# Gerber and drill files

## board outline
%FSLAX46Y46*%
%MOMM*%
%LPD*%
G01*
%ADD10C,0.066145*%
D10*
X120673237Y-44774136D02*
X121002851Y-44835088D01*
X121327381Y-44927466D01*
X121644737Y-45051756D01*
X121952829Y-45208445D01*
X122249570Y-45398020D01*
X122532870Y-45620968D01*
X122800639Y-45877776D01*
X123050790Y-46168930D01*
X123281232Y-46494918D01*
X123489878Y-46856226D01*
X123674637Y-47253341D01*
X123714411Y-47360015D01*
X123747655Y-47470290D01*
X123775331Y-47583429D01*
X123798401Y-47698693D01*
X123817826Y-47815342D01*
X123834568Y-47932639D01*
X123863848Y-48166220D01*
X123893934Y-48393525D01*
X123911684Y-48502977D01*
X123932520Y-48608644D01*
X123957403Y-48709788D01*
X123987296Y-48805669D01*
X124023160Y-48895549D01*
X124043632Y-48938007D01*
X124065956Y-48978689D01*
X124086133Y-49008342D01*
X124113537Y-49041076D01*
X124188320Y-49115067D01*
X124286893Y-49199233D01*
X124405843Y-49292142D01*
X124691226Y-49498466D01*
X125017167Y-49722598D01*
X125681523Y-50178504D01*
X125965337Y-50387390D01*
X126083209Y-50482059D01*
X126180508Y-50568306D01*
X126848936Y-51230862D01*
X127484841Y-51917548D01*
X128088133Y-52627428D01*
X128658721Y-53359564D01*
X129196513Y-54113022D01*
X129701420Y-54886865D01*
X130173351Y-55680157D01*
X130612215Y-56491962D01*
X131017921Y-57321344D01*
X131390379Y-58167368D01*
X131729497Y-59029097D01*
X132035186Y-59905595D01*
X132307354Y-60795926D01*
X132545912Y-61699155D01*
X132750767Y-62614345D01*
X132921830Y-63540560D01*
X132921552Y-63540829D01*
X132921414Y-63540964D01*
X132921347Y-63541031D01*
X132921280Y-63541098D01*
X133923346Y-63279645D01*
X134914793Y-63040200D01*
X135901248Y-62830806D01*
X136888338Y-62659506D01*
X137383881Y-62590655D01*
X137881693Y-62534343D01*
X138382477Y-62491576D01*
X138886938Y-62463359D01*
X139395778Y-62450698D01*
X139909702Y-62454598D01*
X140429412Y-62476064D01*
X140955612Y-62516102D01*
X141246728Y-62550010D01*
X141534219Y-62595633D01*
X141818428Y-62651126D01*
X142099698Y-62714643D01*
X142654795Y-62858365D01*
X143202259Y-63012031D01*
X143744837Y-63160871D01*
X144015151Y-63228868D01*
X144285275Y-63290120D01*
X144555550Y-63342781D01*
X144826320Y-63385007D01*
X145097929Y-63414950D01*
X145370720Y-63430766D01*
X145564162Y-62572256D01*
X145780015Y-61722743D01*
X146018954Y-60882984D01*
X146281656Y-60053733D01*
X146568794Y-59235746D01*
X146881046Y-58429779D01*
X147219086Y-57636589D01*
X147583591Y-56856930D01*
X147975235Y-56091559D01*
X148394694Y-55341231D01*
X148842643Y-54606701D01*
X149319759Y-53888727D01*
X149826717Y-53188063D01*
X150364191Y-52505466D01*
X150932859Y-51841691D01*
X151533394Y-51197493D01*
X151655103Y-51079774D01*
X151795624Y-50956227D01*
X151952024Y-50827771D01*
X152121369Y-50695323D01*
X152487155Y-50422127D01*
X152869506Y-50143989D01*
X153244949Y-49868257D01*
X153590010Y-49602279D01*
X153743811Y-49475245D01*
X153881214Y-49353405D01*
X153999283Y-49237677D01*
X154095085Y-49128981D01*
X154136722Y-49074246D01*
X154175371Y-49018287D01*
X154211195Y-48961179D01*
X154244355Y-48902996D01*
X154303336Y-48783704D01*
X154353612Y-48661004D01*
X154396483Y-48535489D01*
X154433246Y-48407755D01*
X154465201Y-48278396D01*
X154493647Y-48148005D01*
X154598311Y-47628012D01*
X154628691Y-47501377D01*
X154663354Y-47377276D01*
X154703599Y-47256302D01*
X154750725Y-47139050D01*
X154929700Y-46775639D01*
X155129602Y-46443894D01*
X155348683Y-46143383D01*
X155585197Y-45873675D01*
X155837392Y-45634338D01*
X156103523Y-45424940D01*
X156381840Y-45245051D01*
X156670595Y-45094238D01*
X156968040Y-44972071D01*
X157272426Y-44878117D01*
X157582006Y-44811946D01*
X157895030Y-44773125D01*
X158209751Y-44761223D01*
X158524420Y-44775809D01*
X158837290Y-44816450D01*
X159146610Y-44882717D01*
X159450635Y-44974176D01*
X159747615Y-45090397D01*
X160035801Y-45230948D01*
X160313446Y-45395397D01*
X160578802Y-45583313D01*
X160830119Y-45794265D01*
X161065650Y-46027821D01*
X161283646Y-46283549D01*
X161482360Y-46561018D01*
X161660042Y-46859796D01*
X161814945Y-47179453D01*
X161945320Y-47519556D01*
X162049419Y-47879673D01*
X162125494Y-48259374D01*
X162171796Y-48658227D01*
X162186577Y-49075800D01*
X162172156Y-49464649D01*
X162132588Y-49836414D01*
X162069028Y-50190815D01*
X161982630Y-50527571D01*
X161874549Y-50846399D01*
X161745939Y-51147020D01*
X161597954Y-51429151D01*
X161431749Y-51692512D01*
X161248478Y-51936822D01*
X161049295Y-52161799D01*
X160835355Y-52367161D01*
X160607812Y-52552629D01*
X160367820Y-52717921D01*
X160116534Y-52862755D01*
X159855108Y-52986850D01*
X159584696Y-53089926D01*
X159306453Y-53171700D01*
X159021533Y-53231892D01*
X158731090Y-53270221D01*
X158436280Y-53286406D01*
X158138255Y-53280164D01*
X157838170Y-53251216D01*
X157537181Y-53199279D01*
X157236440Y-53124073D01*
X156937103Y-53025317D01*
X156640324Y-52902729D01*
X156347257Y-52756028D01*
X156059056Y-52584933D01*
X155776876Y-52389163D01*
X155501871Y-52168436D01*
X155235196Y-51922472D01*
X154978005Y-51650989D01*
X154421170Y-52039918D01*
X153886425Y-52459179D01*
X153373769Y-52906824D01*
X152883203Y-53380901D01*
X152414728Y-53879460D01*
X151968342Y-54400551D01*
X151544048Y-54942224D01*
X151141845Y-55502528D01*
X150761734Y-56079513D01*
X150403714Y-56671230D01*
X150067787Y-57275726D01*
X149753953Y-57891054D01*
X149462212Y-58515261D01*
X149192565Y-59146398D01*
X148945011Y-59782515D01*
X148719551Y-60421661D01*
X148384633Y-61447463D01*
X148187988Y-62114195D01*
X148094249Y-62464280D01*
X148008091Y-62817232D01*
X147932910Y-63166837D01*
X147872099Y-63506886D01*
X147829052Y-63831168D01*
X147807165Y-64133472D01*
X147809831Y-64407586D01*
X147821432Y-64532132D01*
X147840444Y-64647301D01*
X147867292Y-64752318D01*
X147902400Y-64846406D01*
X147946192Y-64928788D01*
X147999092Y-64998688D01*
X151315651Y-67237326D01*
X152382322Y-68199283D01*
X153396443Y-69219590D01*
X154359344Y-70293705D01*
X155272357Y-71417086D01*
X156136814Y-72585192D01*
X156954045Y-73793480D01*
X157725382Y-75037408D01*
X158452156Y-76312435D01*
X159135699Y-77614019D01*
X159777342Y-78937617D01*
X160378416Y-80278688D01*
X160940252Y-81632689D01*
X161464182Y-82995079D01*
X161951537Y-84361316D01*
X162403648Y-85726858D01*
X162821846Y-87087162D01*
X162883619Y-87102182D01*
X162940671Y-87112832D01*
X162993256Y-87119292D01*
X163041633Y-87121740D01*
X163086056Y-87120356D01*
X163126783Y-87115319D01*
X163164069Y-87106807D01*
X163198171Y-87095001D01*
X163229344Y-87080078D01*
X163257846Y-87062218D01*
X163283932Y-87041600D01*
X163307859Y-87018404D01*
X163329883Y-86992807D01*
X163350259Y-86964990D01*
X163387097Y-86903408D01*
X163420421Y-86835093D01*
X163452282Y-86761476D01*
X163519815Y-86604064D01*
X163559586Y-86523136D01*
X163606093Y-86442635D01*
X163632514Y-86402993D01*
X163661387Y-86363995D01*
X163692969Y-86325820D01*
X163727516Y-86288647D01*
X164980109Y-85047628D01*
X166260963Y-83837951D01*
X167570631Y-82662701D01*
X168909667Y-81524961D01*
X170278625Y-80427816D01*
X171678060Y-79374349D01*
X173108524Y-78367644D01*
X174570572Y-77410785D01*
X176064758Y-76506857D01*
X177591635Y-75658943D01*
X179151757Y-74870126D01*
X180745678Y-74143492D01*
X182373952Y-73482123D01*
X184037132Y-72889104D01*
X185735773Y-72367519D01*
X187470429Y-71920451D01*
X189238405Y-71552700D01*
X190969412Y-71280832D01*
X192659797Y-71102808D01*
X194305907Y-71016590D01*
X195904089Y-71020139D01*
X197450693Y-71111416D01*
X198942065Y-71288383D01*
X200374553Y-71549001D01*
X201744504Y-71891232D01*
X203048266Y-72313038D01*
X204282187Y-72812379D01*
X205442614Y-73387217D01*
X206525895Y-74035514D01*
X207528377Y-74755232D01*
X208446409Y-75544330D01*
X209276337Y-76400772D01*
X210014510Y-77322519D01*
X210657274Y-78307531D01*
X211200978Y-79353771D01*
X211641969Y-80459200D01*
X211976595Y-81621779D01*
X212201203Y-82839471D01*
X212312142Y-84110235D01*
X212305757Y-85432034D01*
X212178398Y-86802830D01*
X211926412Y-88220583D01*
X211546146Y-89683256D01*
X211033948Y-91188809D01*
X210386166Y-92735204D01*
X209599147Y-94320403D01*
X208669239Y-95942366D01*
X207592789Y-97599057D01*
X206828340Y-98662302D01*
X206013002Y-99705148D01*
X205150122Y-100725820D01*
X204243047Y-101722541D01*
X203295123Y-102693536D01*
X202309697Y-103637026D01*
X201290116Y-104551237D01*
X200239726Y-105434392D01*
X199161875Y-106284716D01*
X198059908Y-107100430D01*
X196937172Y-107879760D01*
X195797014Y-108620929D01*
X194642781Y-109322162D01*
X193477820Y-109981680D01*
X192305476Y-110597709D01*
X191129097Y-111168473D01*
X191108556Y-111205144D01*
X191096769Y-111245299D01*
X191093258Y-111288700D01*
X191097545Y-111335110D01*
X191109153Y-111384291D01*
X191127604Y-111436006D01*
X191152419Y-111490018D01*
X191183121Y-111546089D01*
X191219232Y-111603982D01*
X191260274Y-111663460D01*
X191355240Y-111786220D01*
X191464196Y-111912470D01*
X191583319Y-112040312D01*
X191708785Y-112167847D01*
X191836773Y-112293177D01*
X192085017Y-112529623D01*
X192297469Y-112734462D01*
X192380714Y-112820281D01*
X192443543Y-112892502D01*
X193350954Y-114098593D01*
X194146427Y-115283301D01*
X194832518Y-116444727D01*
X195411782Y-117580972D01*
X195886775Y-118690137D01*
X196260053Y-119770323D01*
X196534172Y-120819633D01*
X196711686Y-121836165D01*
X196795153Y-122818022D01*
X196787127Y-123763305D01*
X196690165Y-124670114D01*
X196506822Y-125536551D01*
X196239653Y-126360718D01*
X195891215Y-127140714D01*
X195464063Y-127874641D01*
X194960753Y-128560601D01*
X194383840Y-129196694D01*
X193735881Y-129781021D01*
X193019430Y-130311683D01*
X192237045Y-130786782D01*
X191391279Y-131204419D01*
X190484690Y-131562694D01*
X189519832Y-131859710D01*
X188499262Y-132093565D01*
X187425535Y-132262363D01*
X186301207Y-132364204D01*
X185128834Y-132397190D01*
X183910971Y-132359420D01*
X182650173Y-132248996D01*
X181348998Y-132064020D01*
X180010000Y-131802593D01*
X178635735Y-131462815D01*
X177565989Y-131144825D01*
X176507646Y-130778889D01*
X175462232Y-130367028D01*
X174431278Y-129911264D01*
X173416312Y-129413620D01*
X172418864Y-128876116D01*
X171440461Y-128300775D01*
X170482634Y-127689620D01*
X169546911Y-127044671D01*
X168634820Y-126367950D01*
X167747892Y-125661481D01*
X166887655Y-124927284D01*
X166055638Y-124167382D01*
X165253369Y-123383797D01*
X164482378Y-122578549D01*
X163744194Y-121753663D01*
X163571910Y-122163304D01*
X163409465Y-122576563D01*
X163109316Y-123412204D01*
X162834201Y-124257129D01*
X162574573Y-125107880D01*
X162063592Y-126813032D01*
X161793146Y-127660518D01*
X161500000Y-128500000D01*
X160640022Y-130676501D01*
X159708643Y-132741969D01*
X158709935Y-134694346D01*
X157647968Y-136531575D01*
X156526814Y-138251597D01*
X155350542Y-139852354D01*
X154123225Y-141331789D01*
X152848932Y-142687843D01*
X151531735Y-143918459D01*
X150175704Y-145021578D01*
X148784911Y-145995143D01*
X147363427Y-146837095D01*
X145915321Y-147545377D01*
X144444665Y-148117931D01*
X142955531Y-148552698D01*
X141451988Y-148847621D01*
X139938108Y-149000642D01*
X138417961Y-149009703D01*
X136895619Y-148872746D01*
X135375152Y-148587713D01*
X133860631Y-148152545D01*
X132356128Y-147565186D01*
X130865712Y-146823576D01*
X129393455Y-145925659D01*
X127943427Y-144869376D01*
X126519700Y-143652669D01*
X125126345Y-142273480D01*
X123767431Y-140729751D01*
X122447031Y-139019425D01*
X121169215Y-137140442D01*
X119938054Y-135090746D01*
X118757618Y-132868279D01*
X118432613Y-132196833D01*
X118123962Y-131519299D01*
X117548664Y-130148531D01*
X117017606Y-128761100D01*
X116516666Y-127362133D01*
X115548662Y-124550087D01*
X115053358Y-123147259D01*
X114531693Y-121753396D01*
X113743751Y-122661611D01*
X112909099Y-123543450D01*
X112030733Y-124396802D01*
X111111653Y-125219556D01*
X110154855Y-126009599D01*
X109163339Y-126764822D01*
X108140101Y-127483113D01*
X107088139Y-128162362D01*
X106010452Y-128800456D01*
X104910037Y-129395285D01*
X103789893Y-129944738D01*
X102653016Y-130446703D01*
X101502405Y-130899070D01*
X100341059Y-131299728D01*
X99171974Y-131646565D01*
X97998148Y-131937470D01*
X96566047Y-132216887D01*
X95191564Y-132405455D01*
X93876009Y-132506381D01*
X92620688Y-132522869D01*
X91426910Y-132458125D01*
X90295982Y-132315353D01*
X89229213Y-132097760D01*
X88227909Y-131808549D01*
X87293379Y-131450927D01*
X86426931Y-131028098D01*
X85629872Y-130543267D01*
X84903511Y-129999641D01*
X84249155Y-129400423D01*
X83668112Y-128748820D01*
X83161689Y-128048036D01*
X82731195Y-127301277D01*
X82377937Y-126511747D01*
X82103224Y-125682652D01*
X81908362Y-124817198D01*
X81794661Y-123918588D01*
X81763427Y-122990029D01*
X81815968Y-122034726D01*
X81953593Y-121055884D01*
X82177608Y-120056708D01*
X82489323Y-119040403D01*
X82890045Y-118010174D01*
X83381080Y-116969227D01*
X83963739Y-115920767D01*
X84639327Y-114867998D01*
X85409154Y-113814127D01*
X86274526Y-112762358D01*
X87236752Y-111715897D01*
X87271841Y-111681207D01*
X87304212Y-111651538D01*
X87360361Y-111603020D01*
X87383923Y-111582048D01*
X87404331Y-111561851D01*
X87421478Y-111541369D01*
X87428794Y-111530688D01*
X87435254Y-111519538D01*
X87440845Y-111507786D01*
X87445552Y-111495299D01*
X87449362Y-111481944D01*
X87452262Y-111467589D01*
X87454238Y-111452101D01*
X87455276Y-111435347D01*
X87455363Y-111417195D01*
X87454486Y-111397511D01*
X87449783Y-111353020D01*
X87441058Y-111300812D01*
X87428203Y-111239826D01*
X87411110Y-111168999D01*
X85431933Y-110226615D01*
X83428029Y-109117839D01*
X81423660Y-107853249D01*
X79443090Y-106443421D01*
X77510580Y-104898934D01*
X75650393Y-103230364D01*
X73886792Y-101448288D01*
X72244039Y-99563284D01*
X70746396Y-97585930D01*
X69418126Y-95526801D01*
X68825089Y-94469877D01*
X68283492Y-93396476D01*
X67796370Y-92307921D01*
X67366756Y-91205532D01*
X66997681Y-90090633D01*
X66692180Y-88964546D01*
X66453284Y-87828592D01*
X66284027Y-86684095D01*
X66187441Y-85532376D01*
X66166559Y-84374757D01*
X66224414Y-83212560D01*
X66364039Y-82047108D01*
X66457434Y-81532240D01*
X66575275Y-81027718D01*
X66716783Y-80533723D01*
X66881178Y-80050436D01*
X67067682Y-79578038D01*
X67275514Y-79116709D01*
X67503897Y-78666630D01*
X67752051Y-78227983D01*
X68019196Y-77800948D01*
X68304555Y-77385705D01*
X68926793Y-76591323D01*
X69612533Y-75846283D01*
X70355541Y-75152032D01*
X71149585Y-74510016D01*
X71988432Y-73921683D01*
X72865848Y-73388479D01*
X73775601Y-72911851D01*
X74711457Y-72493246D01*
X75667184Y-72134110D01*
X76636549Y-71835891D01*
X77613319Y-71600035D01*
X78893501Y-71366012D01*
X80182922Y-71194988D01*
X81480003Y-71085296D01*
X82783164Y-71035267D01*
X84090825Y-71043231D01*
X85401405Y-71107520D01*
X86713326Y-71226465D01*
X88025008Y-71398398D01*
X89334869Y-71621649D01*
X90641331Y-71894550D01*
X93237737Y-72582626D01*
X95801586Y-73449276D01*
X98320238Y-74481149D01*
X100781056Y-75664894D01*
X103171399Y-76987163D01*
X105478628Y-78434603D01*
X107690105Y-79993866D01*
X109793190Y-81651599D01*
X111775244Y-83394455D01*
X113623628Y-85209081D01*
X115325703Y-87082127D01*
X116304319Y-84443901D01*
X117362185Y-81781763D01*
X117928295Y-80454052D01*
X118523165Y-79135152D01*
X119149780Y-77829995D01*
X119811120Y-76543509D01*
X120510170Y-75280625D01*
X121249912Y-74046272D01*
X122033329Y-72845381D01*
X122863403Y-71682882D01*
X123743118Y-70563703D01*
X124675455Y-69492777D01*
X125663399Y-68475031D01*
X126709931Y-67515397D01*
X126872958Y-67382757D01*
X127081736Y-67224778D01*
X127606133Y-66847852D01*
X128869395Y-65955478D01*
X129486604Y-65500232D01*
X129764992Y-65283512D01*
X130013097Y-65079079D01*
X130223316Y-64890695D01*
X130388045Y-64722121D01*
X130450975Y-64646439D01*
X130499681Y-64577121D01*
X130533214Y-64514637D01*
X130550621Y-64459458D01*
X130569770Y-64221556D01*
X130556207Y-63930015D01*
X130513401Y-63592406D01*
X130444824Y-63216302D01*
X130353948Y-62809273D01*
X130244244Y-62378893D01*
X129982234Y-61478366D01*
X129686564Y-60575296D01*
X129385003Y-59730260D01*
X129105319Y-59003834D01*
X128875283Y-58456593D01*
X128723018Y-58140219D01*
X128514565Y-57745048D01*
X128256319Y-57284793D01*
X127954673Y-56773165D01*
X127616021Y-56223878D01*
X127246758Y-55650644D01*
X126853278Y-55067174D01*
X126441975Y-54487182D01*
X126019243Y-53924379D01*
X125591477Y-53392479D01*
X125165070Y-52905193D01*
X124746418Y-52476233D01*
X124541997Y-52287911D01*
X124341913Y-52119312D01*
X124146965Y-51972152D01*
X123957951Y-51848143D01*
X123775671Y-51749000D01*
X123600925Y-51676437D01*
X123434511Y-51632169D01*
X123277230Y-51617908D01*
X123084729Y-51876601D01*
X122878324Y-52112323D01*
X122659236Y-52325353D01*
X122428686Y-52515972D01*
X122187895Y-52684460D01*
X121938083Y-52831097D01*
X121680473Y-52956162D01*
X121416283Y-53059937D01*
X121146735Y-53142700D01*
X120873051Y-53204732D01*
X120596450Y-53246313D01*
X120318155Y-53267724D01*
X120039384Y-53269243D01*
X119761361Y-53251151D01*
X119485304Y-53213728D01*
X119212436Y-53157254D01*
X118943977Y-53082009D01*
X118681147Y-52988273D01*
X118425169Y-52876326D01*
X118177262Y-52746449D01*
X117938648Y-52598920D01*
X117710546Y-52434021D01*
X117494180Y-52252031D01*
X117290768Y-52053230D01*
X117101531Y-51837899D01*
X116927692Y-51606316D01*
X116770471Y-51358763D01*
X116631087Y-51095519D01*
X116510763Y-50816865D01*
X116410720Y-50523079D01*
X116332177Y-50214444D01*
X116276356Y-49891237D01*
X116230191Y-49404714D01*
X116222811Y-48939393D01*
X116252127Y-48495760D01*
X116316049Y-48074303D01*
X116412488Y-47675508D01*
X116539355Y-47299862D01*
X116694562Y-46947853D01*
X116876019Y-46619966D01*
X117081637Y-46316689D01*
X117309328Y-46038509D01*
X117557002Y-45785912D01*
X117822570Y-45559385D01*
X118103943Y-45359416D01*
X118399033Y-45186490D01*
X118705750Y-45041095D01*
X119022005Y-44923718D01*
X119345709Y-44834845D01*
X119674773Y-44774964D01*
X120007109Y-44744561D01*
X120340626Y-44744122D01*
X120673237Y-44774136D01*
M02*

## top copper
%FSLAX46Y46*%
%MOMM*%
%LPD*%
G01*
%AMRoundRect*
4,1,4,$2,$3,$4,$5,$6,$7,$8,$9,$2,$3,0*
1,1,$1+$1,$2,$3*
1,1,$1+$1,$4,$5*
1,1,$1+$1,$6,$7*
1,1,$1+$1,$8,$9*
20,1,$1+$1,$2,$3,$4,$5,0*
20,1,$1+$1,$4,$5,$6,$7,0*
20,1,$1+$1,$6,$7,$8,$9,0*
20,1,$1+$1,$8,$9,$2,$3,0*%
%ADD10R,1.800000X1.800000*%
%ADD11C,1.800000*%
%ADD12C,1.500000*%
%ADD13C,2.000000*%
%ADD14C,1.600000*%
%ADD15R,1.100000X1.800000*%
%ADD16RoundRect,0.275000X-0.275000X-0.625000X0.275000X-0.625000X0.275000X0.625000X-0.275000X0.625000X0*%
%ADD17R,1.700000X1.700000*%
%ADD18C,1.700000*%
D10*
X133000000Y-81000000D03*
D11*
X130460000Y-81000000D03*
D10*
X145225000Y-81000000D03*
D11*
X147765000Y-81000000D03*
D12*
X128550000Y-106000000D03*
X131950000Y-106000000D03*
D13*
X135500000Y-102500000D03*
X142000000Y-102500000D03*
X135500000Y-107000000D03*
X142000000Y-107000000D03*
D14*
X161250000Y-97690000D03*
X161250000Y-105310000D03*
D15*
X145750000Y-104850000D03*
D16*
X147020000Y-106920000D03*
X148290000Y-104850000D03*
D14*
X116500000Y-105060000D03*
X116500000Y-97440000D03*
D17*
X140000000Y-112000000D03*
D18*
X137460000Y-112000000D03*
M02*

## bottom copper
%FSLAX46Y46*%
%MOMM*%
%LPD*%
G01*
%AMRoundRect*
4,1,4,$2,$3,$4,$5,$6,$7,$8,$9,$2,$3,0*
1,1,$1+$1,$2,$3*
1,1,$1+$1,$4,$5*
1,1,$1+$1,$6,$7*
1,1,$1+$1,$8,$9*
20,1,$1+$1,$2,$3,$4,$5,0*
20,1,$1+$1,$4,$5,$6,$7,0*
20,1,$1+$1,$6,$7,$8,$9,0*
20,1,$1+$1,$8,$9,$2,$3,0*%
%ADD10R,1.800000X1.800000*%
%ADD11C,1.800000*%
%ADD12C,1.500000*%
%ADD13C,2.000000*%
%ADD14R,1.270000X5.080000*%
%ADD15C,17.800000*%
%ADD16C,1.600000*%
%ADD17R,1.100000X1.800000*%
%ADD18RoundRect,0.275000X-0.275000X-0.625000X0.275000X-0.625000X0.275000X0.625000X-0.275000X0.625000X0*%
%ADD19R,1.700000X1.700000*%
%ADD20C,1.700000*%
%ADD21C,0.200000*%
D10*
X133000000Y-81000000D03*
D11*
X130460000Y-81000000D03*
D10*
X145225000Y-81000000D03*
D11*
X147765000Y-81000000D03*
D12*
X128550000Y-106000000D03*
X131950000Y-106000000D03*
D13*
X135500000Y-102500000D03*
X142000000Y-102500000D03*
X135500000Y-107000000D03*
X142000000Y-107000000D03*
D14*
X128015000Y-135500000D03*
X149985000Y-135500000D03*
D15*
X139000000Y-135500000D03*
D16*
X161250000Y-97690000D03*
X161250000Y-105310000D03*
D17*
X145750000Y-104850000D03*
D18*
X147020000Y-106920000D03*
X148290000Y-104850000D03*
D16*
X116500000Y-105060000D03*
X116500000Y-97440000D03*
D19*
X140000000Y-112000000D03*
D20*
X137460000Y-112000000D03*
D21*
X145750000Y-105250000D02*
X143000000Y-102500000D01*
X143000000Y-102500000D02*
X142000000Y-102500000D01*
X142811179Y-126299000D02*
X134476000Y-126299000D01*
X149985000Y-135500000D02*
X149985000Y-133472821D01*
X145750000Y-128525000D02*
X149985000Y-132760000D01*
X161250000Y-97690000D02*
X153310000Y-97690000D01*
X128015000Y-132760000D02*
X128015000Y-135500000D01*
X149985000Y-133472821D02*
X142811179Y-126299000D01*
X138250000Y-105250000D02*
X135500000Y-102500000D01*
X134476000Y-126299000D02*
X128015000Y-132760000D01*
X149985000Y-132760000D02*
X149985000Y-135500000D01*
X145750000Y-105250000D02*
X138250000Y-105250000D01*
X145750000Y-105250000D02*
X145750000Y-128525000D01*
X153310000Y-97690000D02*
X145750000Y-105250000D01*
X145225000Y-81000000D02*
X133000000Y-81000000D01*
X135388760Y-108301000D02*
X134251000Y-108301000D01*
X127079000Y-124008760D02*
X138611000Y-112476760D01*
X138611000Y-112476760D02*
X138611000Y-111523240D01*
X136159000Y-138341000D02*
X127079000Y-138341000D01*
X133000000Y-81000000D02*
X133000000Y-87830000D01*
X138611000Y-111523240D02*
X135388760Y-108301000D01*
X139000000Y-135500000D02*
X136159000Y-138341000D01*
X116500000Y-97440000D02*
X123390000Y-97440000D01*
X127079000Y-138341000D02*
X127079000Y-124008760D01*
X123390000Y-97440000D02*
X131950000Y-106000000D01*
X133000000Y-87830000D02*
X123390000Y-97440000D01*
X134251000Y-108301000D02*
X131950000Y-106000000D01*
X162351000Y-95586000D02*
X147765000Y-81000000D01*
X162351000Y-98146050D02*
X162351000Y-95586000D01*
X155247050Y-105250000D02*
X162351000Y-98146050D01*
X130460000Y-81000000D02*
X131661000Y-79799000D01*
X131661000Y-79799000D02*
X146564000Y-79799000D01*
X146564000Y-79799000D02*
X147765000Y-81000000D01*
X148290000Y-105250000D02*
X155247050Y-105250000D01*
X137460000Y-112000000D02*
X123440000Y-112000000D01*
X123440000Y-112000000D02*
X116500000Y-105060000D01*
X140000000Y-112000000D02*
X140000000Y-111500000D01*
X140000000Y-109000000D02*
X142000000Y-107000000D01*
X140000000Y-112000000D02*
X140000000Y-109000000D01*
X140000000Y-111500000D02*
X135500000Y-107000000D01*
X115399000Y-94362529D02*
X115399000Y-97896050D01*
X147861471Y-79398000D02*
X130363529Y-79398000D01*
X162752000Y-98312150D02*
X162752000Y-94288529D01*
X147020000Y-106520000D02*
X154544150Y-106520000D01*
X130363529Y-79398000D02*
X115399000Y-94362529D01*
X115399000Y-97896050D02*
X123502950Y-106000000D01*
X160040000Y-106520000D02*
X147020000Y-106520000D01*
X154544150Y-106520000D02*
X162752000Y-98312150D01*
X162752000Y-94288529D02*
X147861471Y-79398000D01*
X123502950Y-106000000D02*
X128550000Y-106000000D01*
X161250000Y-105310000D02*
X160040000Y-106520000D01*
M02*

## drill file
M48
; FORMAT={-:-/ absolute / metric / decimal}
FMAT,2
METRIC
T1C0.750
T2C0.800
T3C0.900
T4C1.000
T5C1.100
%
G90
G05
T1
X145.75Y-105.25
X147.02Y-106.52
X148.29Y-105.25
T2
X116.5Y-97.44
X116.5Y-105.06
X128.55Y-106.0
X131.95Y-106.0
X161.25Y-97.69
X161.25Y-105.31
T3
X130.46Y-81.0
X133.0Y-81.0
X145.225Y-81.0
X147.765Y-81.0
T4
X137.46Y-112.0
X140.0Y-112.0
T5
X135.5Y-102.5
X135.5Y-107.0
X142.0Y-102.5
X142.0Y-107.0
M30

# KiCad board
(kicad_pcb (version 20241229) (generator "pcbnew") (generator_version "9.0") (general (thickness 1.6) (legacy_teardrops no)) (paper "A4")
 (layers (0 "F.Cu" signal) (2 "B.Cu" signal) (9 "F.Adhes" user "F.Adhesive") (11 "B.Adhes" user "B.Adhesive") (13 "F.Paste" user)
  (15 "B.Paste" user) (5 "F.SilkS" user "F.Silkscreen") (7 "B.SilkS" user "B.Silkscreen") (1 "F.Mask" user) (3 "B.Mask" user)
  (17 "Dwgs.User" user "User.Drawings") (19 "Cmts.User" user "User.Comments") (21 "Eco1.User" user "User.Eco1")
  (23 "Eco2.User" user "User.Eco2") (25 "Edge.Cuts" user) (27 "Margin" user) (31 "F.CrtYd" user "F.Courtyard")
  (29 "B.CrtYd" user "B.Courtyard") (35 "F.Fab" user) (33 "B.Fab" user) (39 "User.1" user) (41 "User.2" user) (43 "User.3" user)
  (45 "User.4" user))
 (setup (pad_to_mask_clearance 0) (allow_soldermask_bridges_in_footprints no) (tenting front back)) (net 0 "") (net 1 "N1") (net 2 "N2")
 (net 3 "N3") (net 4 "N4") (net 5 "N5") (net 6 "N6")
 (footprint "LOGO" (layer "F.Cu") (at 139.25 97.25)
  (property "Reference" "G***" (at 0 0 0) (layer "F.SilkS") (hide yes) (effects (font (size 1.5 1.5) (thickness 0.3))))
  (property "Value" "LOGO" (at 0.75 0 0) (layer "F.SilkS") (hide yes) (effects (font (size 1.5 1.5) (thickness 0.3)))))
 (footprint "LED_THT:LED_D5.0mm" (layer "F.Cu") (at 133 81 180)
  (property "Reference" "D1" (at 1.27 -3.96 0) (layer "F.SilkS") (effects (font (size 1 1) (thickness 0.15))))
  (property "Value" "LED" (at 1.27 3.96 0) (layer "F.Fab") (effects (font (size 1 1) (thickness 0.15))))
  (pad "1" thru_hole rect (at 0 0 180) (size 1.8 1.8) (drill 0.9) (layers "*.Cu" "*.Mask") (remove_unused_layers no) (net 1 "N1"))
  (pad "2" thru_hole circle (at 2.54 0 180) (size 1.8 1.8) (drill 0.9) (layers "*.Cu" "*.Mask") (remove_unused_layers no) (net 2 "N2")))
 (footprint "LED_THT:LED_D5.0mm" (layer "F.Cu") (at 145.225 81)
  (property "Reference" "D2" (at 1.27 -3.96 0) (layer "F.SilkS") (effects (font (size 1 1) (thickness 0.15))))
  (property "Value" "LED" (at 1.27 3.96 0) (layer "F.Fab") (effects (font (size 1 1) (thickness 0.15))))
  (pad "1" thru_hole rect (at 0 0) (size 1.8 1.8) (drill 0.9) (layers "*.Cu" "*.Mask") (remove_unused_layers no) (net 1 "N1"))
  (pad "2" thru_hole circle (at 2.54 0) (size 1.8 1.8) (drill 0.9) (layers "*.Cu" "*.Mask") (remove_unused_layers no) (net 2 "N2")))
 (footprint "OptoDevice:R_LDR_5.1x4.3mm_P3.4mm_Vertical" (layer "F.Cu") (at 128.55 106)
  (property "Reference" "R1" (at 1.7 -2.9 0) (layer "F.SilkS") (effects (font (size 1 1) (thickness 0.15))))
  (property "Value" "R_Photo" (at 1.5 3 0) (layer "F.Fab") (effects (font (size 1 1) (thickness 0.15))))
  (pad "1" thru_hole circle (at 0 0) (size 1.5 1.5) (drill 0.8) (layers "*.Cu" "*.Mask") (remove_unused_layers no) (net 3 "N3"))
  (pad "2" thru_hole circle (at 3.4 0) (size 1.5 1.5) (drill 0.8) (layers "*.Cu" "*.Mask") (remove_unused_layers no) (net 1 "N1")))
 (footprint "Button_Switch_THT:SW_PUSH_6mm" (layer "F.Cu") (at 135.5 102.5)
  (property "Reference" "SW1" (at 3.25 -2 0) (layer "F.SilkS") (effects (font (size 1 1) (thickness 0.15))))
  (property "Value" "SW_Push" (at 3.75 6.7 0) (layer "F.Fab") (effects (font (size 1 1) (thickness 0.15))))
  (pad "1" thru_hole circle (at 0 0 90) (size 2 2) (drill 1.1) (layers "*.Cu" "*.Mask") (remove_unused_layers no) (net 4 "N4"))
  (pad "1" thru_hole circle (at 6.5 0 90) (size 2 2) (drill 1.1) (layers "*.Cu" "*.Mask") (remove_unused_layers no) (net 4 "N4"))
  (pad "2" thru_hole circle (at 0 4.5 90) (size 2 2) (drill 1.1) (layers "*.Cu" "*.Mask") (remove_unused_layers no) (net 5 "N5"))
  (pad "2" thru_hole circle (at 6.5 4.5 90) (size 2 2) (drill 1.1) (layers "*.Cu" "*.Mask") (remove_unused_layers no) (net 5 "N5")))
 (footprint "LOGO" (layer "B.Cu") (at 102.5 124 180)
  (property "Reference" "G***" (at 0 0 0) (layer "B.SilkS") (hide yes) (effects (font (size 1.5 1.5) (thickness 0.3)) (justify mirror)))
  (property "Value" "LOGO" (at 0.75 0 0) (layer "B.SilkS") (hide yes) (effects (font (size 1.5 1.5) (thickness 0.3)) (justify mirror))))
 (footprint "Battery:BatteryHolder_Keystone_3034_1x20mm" (layer "B.Cu") (at 139 135.5)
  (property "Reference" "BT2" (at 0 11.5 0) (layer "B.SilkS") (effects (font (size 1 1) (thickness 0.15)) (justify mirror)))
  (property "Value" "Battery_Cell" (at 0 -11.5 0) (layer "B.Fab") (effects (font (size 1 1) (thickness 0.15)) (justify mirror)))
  (pad "1" smd rect (at -10.985 0) (size 1.27 5.08) (layers "B.Cu" "B.Mask" "B.Paste") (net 4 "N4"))
  (pad "1" smd rect (at 10.985 0) (size 1.27 5.08) (layers "B.Cu" "B.Mask" "B.Paste") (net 4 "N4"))
  (pad "2" smd circle (at 0 0) (size 17.8 17.8) (layers "B.Cu" "B.Mask") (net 1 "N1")))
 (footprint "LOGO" (layer "B.Cu") (at 183.5 123.75 180)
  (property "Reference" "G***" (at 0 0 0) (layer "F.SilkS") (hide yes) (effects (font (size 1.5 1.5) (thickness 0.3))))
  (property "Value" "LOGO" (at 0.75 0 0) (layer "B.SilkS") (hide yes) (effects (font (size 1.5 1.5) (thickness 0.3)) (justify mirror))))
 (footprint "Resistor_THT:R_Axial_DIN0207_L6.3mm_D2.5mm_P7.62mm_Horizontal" (layer "B.Cu") (at 161.25 97.69 -90)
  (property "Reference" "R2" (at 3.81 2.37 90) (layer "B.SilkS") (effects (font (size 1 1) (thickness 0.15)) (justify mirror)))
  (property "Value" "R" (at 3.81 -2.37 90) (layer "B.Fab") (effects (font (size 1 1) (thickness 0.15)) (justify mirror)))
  (pad "1" thru_hole circle (at 0 0 270) (size 1.6 1.6) (drill 0.8) (layers "*.Cu" "*.Mask") (remove_unused_layers no) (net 4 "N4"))
  (pad "2" thru_hole circle (at 7.62 0 270) (size 1.6 1.6) (drill 0.8) (layers "*.Cu" "*.Mask") (remove_unused_layers no) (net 3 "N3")))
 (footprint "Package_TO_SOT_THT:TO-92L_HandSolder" (layer "B.Cu") (at 145.75 105.25)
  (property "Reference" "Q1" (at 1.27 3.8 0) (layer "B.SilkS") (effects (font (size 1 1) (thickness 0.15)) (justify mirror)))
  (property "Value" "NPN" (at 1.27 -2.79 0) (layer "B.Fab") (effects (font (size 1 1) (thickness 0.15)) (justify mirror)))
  (pad "1" thru_hole rect (at 0 0) (size 1.1 1.8) (drill 0.75 (offset 0 -0.4)) (layers "*.Cu" "*.Mask") (remove_unused_layers no)
   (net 4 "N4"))
  (pad "2" thru_hole roundrect (at 1.27 1.27) (size 1.1 1.8) (drill 0.75 (offset 0 0.4)) (layers "*.Cu" "*.Mask") (remove_unused_layers no)
   (roundrect_rratio 0.25) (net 3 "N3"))
  (pad "3" thru_hole roundrect (at 2.54 0) (size 1.1 1.8) (drill 0.75 (offset 0 -0.4)) (layers "*.Cu" "*.Mask") (remove_unused_layers no)
   (roundrect_rratio 0.25) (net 2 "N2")))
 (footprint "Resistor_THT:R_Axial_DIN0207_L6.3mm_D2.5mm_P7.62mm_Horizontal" (layer "B.Cu") (at 116.5 105.06 90)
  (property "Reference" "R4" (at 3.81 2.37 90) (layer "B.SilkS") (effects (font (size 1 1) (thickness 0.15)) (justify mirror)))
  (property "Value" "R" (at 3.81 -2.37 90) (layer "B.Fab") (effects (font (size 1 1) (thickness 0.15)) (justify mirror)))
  (pad "1" thru_hole circle (at 0 0 90) (size 1.6 1.6) (drill 0.8) (layers "*.Cu" "*.Mask") (remove_unused_layers no) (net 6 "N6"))
  (pad "2" thru_hole circle (at 7.62 0 90) (size 1.6 1.6) (drill 0.8) (layers "*.Cu" "*.Mask") (remove_unused_layers no) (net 1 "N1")))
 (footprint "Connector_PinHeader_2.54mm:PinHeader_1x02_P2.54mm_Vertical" (layer "B.Cu") (at 140 112 90)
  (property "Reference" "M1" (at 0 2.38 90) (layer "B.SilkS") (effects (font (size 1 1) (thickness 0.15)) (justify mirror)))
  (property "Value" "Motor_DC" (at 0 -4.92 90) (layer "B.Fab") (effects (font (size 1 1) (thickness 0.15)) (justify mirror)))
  (pad "1" thru_hole rect (at 0 0 90) (size 1.7 1.7) (drill 1) (layers "*.Cu" "*.Mask") (remove_unused_layers no) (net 5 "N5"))
  (pad "2" thru_hole circle (at 0 -2.54 90) (size 1.7 1.7) (drill 1) (layers "*.Cu" "*.Mask") (remove_unused_layers no) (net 6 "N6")))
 (gr_poly
  (pts (xy 120.673237 44.774136) (xy 121.002851 44.835088) (xy 121.327381 44.927466) (xy 121.644737 45.051756) (xy 121.952829 45.208445)
   (xy 122.24957 45.39802) (xy 122.53287 45.620968) (xy 122.800639 45.877776) (xy 123.05079 46.16893) (xy 123.281232 46.494918)
   (xy 123.489878 46.856226) (xy 123.674637 47.253341) (xy 123.714411 47.360015) (xy 123.747655 47.47029) (xy 123.775331 47.583429)
   (xy 123.798401 47.698693) (xy 123.817826 47.815342) (xy 123.834568 47.932639) (xy 123.863848 48.16622) (xy 123.893934 48.393525)
   (xy 123.911684 48.502977) (xy 123.93252 48.608644) (xy 123.957403 48.709788) (xy 123.987296 48.805669) (xy 124.02316 48.895549)
   (xy 124.043632 48.938007) (xy 124.065956 48.978689) (xy 124.086133 49.008342) (xy 124.113537 49.041076) (xy 124.18832 49.115067)
   (xy 124.286893 49.199233) (xy 124.405843 49.292142) (xy 124.691226 49.498466) (xy 125.017167 49.722598) (xy 125.681523 50.178504)
   (xy 125.965337 50.38739) (xy 126.083209 50.482059) (xy 126.180508 50.568306) (xy 126.848936 51.230862) (xy 127.484841 51.917548)
   (xy 128.088133 52.627428) (xy 128.658721 53.359564) (xy 129.196513 54.113022) (xy 129.70142 54.886865) (xy 130.173351 55.680157)
   (xy 130.612215 56.491962) (xy 131.017921 57.321344) (xy 131.390379 58.167368) (xy 131.729497 59.029097) (xy 132.035186 59.905595)
   (xy 132.307354 60.795926) (xy 132.545912 61.699155) (xy 132.750767 62.614345) (xy 132.92183 63.54056) (xy 132.921552 63.540829)
   (xy 132.921414 63.540964) (xy 132.921347 63.541031) (xy 132.92128 63.541098) (xy 133.923346 63.279645) (xy 134.914793 63.0402)
   (xy 135.901248 62.830806) (xy 136.888338 62.659506) (xy 137.383881 62.590655) (xy 137.881693 62.534343) (xy 138.382477 62.491576)
   (xy 138.886938 62.463359) (xy 139.395778 62.450698) (xy 139.909702 62.454598) (xy 140.429412 62.476064) (xy 140.955612 62.516102)
   (xy 141.246728 62.55001) (xy 141.534219 62.595633) (xy 141.818428 62.651126) (xy 142.099698 62.714643) (xy 142.654795 62.858365)
   (xy 143.202259 63.012031) (xy 143.744837 63.160871) (xy 144.015151 63.228868) (xy 144.285275 63.29012) (xy 144.55555 63.342781)
   (xy 144.82632 63.385007) (xy 145.097929 63.41495) (xy 145.37072 63.430766) (xy 145.564162 62.572256) (xy 145.780015 61.722743)
   (xy 146.018954 60.882984) (xy 146.281656 60.053733) (xy 146.568794 59.235746) (xy 146.881046 58.429779) (xy 147.219086 57.636589)
   (xy 147.583591 56.85693) (xy 147.975235 56.091559) (xy 148.394694 55.341231) (xy 148.842643 54.606701) (xy 149.319759 53.888727)
   (xy 149.826717 53.188063) (xy 150.364191 52.505466) (xy 150.932859 51.841691) (xy 151.533394 51.197493) (xy 151.655103 51.079774)
   (xy 151.795624 50.956227) (xy 151.952024 50.827771) (xy 152.121369 50.695323) (xy 152.487155 50.422127) (xy 152.869506 50.143989)
   (xy 153.244949 49.868257) (xy 153.59001 49.602279) (xy 153.743811 49.475245) (xy 153.881214 49.353405) (xy 153.999283 49.237677)
   (xy 154.095085 49.128981) (xy 154.136722 49.074246) (xy 154.175371 49.018287) (xy 154.211195 48.961179) (xy 154.244355 48.902996)
   (xy 154.303336 48.783704) (xy 154.353612 48.661004) (xy 154.396483 48.535489) (xy 154.433246 48.407755) (xy 154.465201 48.278396)
   (xy 154.493647 48.148005) (xy 154.598311 47.628012) (xy 154.628691 47.501377) (xy 154.663354 47.377276) (xy 154.703599 47.256302)
   (xy 154.750725 47.13905) (xy 154.9297 46.775639) (xy 155.129602 46.443894) (xy 155.348683 46.143383) (xy 155.585197 45.873675)
   (xy 155.837392 45.634338) (xy 156.103523 45.42494) (xy 156.38184 45.245051) (xy 156.670595 45.094238) (xy 156.96804 44.972071)
   (xy 157.272426 44.878117) (xy 157.582006 44.811946) (xy 157.89503 44.773125) (xy 158.209751 44.761223) (xy 158.52442 44.775809)
   (xy 158.83729 44.81645) (xy 159.14661 44.882717) (xy 159.450635 44.974176) (xy 159.747615 45.090397) (xy 160.035801 45.230948)
   (xy 160.313446 45.395397) (xy 160.578802 45.583313) (xy 160.830119 45.794265) (xy 161.06565 46.027821) (xy 161.283646 46.283549)
   (xy 161.48236 46.561018) (xy 161.660042 46.859796) (xy 161.814945 47.179453) (xy 161.94532 47.519556) (xy 162.049419 47.879673)
   (xy 162.125494 48.259374) (xy 162.171796 48.658227) (xy 162.186577 49.0758) (xy 162.172156 49.464649) (xy 162.132588 49.836414)
   (xy 162.069028 50.190815) (xy 161.98263 50.527571) (xy 161.874549 50.846399) (xy 161.745939 51.14702) (xy 161.597954 51.429151)
   (xy 161.431749 51.692512) (xy 161.248478 51.936822) (xy 161.049295 52.161799) (xy 160.835355 52.367161) (xy 160.607812 52.552629)
   (xy 160.36782 52.717921) (xy 160.116534 52.862755) (xy 159.855108 52.98685) (xy 159.584696 53.089926) (xy 159.306453 53.1717)
   (xy 159.021533 53.231892) (xy 158.73109 53.270221) (xy 158.43628 53.286406) (xy 158.138255 53.280164) (xy 157.83817 53.251216)
   (xy 157.537181 53.199279) (xy 157.23644 53.124073) (xy 156.937103 53.025317) (xy 156.640324 52.902729) (xy 156.347257 52.756028)
   (xy 156.059056 52.584933) (xy 155.776876 52.389163) (xy 155.501871 52.168436) (xy 155.235196 51.922472) (xy 154.978005 51.650989)
   (xy 154.42117 52.039918) (xy 153.886425 52.459179) (xy 153.373769 52.906824) (xy 152.883203 53.380901) (xy 152.414728 53.87946)
   (xy 151.968342 54.400551) (xy 151.544048 54.942224) (xy 151.141845 55.502528) (xy 150.761734 56.079513) (xy 150.403714 56.67123)
   (xy 150.067787 57.275726) (xy 149.753953 57.891054) (xy 149.462212 58.515261) (xy 149.192565 59.146398) (xy 148.945011 59.782515)
   (xy 148.719551 60.421661) (xy 148.384633 61.447463) (xy 148.187988 62.114195) (xy 148.094249 62.46428) (xy 148.008091 62.817232)
   (xy 147.93291 63.166837) (xy 147.872099 63.506886) (xy 147.829052 63.831168) (xy 147.807165 64.133472) (xy 147.809831 64.407586)
   (xy 147.821432 64.532132) (xy 147.840444 64.647301) (xy 147.867292 64.752318) (xy 147.9024 64.846406) (xy 147.946192 64.928788)
   (xy 147.999092 64.998688) (xy 151.315651 67.237326) (xy 152.382322 68.199283) (xy 153.396443 69.21959) (xy 154.359344 70.293705)
   (xy 155.272357 71.417086) (xy 156.136814 72.585192) (xy 156.954045 73.79348) (xy 157.725382 75.037408) (xy 158.452156 76.312435)
   (xy 159.135699 77.614019) (xy 159.777342 78.937617) (xy 160.378416 80.278688) (xy 160.940252 81.632689) (xy 161.464182 82.995079)
   (xy 161.951537 84.361316) (xy 162.403648 85.726858) (xy 162.821846 87.087162) (xy 162.883619 87.102182) (xy 162.940671 87.112832)
   (xy 162.993256 87.119292) (xy 163.041633 87.12174) (xy 163.086056 87.120356) (xy 163.126783 87.115319) (xy 163.164069 87.106807)
   (xy 163.198171 87.095001) (xy 163.229344 87.080078) (xy 163.257846 87.062218) (xy 163.283932 87.0416) (xy 163.307859 87.018404)
   (xy 163.329883 86.992807) (xy 163.350259 86.96499) (xy 163.387097 86.903408) (xy 163.420421 86.835093) (xy 163.452282 86.761476)
   (xy 163.519815 86.604064) (xy 163.559586 86.523136) (xy 163.606093 86.442635) (xy 163.632514 86.402993) (xy 163.661387 86.363995)
   (xy 163.692969 86.32582) (xy 163.727516 86.288647) (xy 164.980109 85.047628) (xy 166.260963 83.837951) (xy 167.570631 82.662701)
   (xy 168.909667 81.524961) (xy 170.278625 80.427816) (xy 171.67806 79.374349) (xy 173.108524 78.367644) (xy 174.570572 77.410785)
   (xy 176.064758 76.506857) (xy 177.591635 75.658943) (xy 179.151757 74.870126) (xy 180.745678 74.143492) (xy 182.373952 73.482123)
   (xy 184.037132 72.889104) (xy 185.735773 72.367519) (xy 187.470429 71.920451) (xy 189.238405 71.5527) (xy 190.969412 71.280832)
   (xy 192.659797 71.102808) (xy 194.305907 71.01659) (xy 195.904089 71.020139) (xy 197.450693 71.111416) (xy 198.942065 71.288383)
   (xy 200.374553 71.549001) (xy 201.744504 71.891232) (xy 203.048266 72.313038) (xy 204.282187 72.812379) (xy 205.442614 73.387217)
   (xy 206.525895 74.035514) (xy 207.528377 74.755232) (xy 208.446409 75.54433) (xy 209.276337 76.400772) (xy 210.01451 77.322519)
   (xy 210.657274 78.307531) (xy 211.200978 79.353771) (xy 211.641969 80.4592) (xy 211.976595 81.621779) (xy 212.201203 82.839471)
   (xy 212.312142 84.110235) (xy 212.305757 85.432034) (xy 212.178398 86.80283) (xy 211.926412 88.220583) (xy 211.546146 89.683256)
   (xy 211.033948 91.188809) (xy 210.386166 92.735204) (xy 209.599147 94.320403) (xy 208.669239 95.942366) (xy 207.592789 97.599057)
   (xy 206.82834 98.662302) (xy 206.013002 99.705148) (xy 205.150122 100.72582) (xy 204.243047 101.722541) (xy 203.295123 102.693536)
   (xy 202.309697 103.637026) (xy 201.290116 104.551237) (xy 200.239726 105.434392) (xy 199.161875 106.284716) (xy 198.059908 107.10043)
   (xy 196.937172 107.87976) (xy 195.797014 108.620929) (xy 194.642781 109.322162) (xy 193.47782 109.98168) (xy 192.305476 110.597709)
   (xy 191.129097 111.168473) (xy 191.108556 111.205144) (xy 191.096769 111.245299) (xy 191.093258 111.2887) (xy 191.097545 111.33511)
   (xy 191.109153 111.384291) (xy 191.127604 111.436006) (xy 191.152419 111.490018) (xy 191.183121 111.546089) (xy 191.219232 111.603982)
   (xy 191.260274 111.66346) (xy 191.35524 111.78622) (xy 191.464196 111.91247) (xy 191.583319 112.040312) (xy 191.708785 112.167847)
   (xy 191.836773 112.293177) (xy 192.085017 112.529623) (xy 192.297469 112.734462) (xy 192.380714 112.820281) (xy 192.443543 112.892502)
   (xy 193.350954 114.098593) (xy 194.146427 115.283301) (xy 194.832518 116.444727) (xy 195.411782 117.580972) (xy 195.886775 118.690137)
   (xy 196.260053 119.770323) (xy 196.534172 120.819633) (xy 196.711686 121.836165) (xy 196.795153 122.818022) (xy 196.787127 123.763305)
   (xy 196.690165 124.670114) (xy 196.506822 125.536551) (xy 196.239653 126.360718) (xy 195.891215 127.140714) (xy 195.464063 127.874641)
   (xy 194.960753 128.560601) (xy 194.38384 129.196694) (xy 193.735881 129.781021) (xy 193.01943 130.311683) (xy 192.237045 130.786782)
   (xy 191.391279 131.204419) (xy 190.48469 131.562694) (xy 189.519832 131.85971) (xy 188.499262 132.093565) (xy 187.425535 132.262363)
   (xy 186.301207 132.364204) (xy 185.128834 132.39719) (xy 183.910971 132.35942) (xy 182.650173 132.248996) (xy 181.348998 132.06402)
   (xy 180.01 131.802593) (xy 178.635735 131.462815) (xy 177.565989 131.144825) (xy 176.507646 130.778889) (xy 175.462232 130.367028)
   (xy 174.431278 129.911264) (xy 173.416312 129.41362) (xy 172.418864 128.876116) (xy 171.440461 128.300775) (xy 170.482634 127.68962)
   (xy 169.546911 127.044671) (xy 168.63482 126.36795) (xy 167.747892 125.661481) (xy 166.887655 124.927284) (xy 166.055638 124.167382)
   (xy 165.253369 123.383797) (xy 164.482378 122.578549) (xy 163.744194 121.753663) (xy 163.57191 122.163304) (xy 163.409465 122.576563)
   (xy 163.109316 123.412204) (xy 162.834201 124.257129) (xy 162.574573 125.10788) (xy 162.063592 126.813032) (xy 161.793146 127.660518)
   (xy 161.5 128.5) (xy 160.640022 130.676501) (xy 159.708643 132.741969) (xy 158.709935 134.694346) (xy 157.647968 136.531575)
   (xy 156.526814 138.251597) (xy 155.350542 139.852354) (xy 154.123225 141.331789) (xy 152.848932 142.687843) (xy 151.531735 143.918459)
   (xy 150.175704 145.021578) (xy 148.784911 145.995143) (xy 147.363427 146.837095) (xy 145.915321 147.545377) (xy 144.444665 148.117931)
   (xy 142.955531 148.552698) (xy 141.451988 148.847621) (xy 139.938108 149.000642) (xy 138.417961 149.009703) (xy 136.895619 148.872746)
   (xy 135.375152 148.587713) (xy 133.860631 148.152545) (xy 132.356128 147.565186) (xy 130.865712 146.823576) (xy 129.393455 145.925659)
   (xy 127.943427 144.869376) (xy 126.5197 143.652669) (xy 125.126345 142.27348) (xy 123.767431 140.729751) (xy 122.447031 139.019425)
   (xy 121.169215 137.140442) (xy 119.938054 135.090746) (xy 118.757618 132.868279) (xy 118.432613 132.196833) (xy 118.123962 131.519299)
   (xy 117.548664 130.148531) (xy 117.017606 128.7611) (xy 116.516666 127.362133) (xy 115.548662 124.550087) (xy 115.053358 123.147259)
   (xy 114.531693 121.753396) (xy 113.743751 122.661611) (xy 112.909099 123.54345) (xy 112.030733 124.396802) (xy 111.111653 125.219556)
   (xy 110.154855 126.009599) (xy 109.163339 126.764822) (xy 108.140101 127.483113) (xy 107.088139 128.162362) (xy 106.010452 128.800456)
   (xy 104.910037 129.395285) (xy 103.789893 129.944738) (xy 102.653016 130.446703) (xy 101.502405 130.89907) (xy 100.341059 131.299728)
   (xy 99.171974 131.646565) (xy 97.998148 131.93747) (xy 96.566047 132.216887) (xy 95.191564 132.405455) (xy 93.876009 132.506381)
   (xy 92.620688 132.522869) (xy 91.42691 132.458125) (xy 90.295982 132.315353) (xy 89.229213 132.09776) (xy 88.227909 131.808549)
   (xy 87.293379 131.450927) (xy 86.426931 131.028098) (xy 85.629872 130.543267) (xy 84.903511 129.999641) (xy 84.249155 129.400423)
   (xy 83.668112 128.74882) (xy 83.161689 128.048036) (xy 82.731195 127.301277) (xy 82.377937 126.511747) (xy 82.103224 125.682652)
   (xy 81.908362 124.817198) (xy 81.794661 123.918588) (xy 81.763427 122.990029) (xy 81.815968 122.034726) (xy 81.953593 121.055884)
   (xy 82.177608 120.056708) (xy 82.489323 119.040403) (xy 82.890045 118.010174) (xy 83.38108 116.969227) (xy 83.963739 115.920767)
   (xy 84.639327 114.867998) (xy 85.409154 113.814127) (xy 86.274526 112.762358) (xy 87.236752 111.715897) (xy 87.271841 111.681207)
   (xy 87.304212 111.651538) (xy 87.360361 111.60302) (xy 87.383923 111.582048) (xy 87.404331 111.561851) (xy 87.421478 111.541369)
   (xy 87.428794 111.530688) (xy 87.435254 111.519538) (xy 87.440845 111.507786) (xy 87.445552 111.495299) (xy 87.449362 111.481944)
   (xy 87.452262 111.467589) (xy 87.454238 111.452101) (xy 87.455276 111.435347) (xy 87.455363 111.417195) (xy 87.454486 111.397511)
   (xy 87.449783 111.35302) (xy 87.441058 111.300812) (xy 87.428203 111.239826) (xy 87.41111 111.168999) (xy 85.431933 110.226615)
   (xy 83.428029 109.117839) (xy 81.42366 107.853249) (xy 79.44309 106.443421) (xy 77.51058 104.898934) (xy 75.650393 103.230364)
   (xy 73.886792 101.448288) (xy 72.244039 99.563284) (xy 70.746396 97.58593) (xy 69.418126 95.526801) (xy 68.825089 94.469877)
   (xy 68.283492 93.396476) (xy 67.79637 92.307921) (xy 67.366756 91.205532) (xy 66.997681 90.090633) (xy 66.69218 88.964546)
   (xy 66.453284 87.828592) (xy 66.284027 86.684095) (xy 66.187441 85.532376) (xy 66.166559 84.374757) (xy 66.224414 83.21256)
   (xy 66.364039 82.047108) (xy 66.457434 81.53224) (xy 66.575275 81.027718) (xy 66.716783 80.533723) (xy 66.881178 80.050436)
   (xy 67.067682 79.578038) (xy 67.275514 79.116709) (xy 67.503897 78.66663) (xy 67.752051 78.227983) (xy 68.019196 77.800948)
   (xy 68.304555 77.385705) (xy 68.926793 76.591323) (xy 69.612533 75.846283) (xy 70.355541 75.152032) (xy 71.149585 74.510016)
   (xy 71.988432 73.921683) (xy 72.865848 73.388479) (xy 73.775601 72.911851) (xy 74.711457 72.493246) (xy 75.667184 72.13411)
   (xy 76.636549 71.835891) (xy 77.613319 71.600035) (xy 78.893501 71.366012) (xy 80.182922 71.194988) (xy 81.480003 71.085296)
   (xy 82.783164 71.035267) (xy 84.090825 71.043231) (xy 85.401405 71.10752) (xy 86.713326 71.226465) (xy 88.025008 71.398398)
   (xy 89.334869 71.621649) (xy 90.641331 71.89455) (xy 93.237737 72.582626) (xy 95.801586 73.449276) (xy 98.320238 74.481149)
   (xy 100.781056 75.664894) (xy 103.171399 76.987163) (xy 105.478628 78.434603) (xy 107.690105 79.993866) (xy 109.79319 81.651599)
   (xy 111.775244 83.394455) (xy 113.623628 85.209081) (xy 115.325703 87.082127) (xy 116.304319 84.443901) (xy 117.362185 81.781763)
   (xy 117.928295 80.454052) (xy 118.523165 79.135152) (xy 119.14978 77.829995) (xy 119.81112 76.543509) (xy 120.51017 75.280625)
   (xy 121.249912 74.046272) (xy 122.033329 72.845381) (xy 122.863403 71.682882) (xy 123.743118 70.563703) (xy 124.675455 69.492777)
   (xy 125.663399 68.475031) (xy 126.709931 67.515397) (xy 126.872958 67.382757) (xy 127.081736 67.224778) (xy 127.606133 66.847852)
   (xy 128.869395 65.955478) (xy 129.486604 65.500232) (xy 129.764992 65.283512) (xy 130.013097 65.079079) (xy 130.223316 64.890695)
   (xy 130.388045 64.722121) (xy 130.450975 64.646439) (xy 130.499681 64.577121) (xy 130.533214 64.514637) (xy 130.550621 64.459458)
   (xy 130.56977 64.221556) (xy 130.556207 63.930015) (xy 130.513401 63.592406) (xy 130.444824 63.216302) (xy 130.353948 62.809273)
   (xy 130.244244 62.378893) (xy 129.982234 61.478366) (xy 129.686564 60.575296) (xy 129.385003 59.73026) (xy 129.105319 59.003834)
   (xy 128.875283 58.456593) (xy 128.723018 58.140219) (xy 128.514565 57.745048) (xy 128.256319 57.284793) (xy 127.954673 56.773165)
   (xy 127.616021 56.223878) (xy 127.246758 55.650644) (xy 126.853278 55.067174) (xy 126.441975 54.487182) (xy 126.019243 53.924379)
   (xy 125.591477 53.392479) (xy 125.16507 52.905193) (xy 124.746418 52.476233) (xy 124.541997 52.287911) (xy 124.341913 52.119312)
   (xy 124.146965 51.972152) (xy 123.957951 51.848143) (xy 123.775671 51.749) (xy 123.600925 51.676437) (xy 123.434511 51.632169)
   (xy 123.27723 51.617908) (xy 123.084729 51.876601) (xy 122.878324 52.112323) (xy 122.659236 52.325353) (xy 122.428686 52.515972)
   (xy 122.187895 52.68446) (xy 121.938083 52.831097) (xy 121.680473 52.956162) (xy 121.416283 53.059937) (xy 121.146735 53.1427)
   (xy 120.873051 53.204732) (xy 120.59645 53.246313) (xy 120.318155 53.267724) (xy 120.039384 53.269243) (xy 119.761361 53.251151)
   (xy 119.485304 53.213728) (xy 119.212436 53.157254) (xy 118.943977 53.082009) (xy 118.681147 52.988273) (xy 118.425169 52.876326)
   (xy 118.177262 52.746449) (xy 117.938648 52.59892) (xy 117.710546 52.434021) (xy 117.49418 52.252031) (xy 117.290768 52.05323)
   (xy 117.101531 51.837899) (xy 116.927692 51.606316) (xy 116.770471 51.358763) (xy 116.631087 51.095519) (xy 116.510763 50.816865)
   (xy 116.41072 50.523079) (xy 116.332177 50.214444) (xy 116.276356 49.891237) (xy 116.230191 49.404714) (xy 116.222811 48.939393)
   (xy 116.252127 48.49576) (xy 116.316049 48.074303) (xy 116.412488 47.675508) (xy 116.539355 47.299862) (xy 116.694562 46.947853)
   (xy 116.876019 46.619966) (xy 117.081637 46.316689) (xy 117.309328 46.038509) (xy 117.557002 45.785912) (xy 117.82257 45.559385)
   (xy 118.103943 45.359416) (xy 118.399033 45.18649) (xy 118.70575 45.041095) (xy 119.022005 44.923718) (xy 119.345709 44.834845)
   (xy 119.674773 44.774964) (xy 120.007109 44.744561) (xy 120.340626 44.744122))
  (stroke (width 0.066145) (type solid)) (fill no) (layer "Edge.Cuts"))
 (segment (start 145.75 105.25) (end 143 102.5) (width 0.2) (layer "B.Cu") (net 4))
 (segment (start 143 102.5) (end 142 102.5) (width 0.2) (layer "B.Cu") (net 4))
 (segment (start 142.811179 126.299) (end 134.476 126.299) (width 0.2) (layer "B.Cu") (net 4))
 (segment (start 149.985 135.5) (end 149.985 133.472821) (width 0.2) (layer "B.Cu") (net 4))
 (segment (start 145.75 128.525) (end 149.985 132.76) (width 0.2) (layer "B.Cu") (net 4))
 (segment (start 161.25 97.69) (end 153.31 97.69) (width 0.2) (layer "B.Cu") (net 4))
 (segment (start 128.015 132.76) (end 128.015 135.5) (width 0.2) (layer "B.Cu") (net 4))
 (segment (start 149.985 133.472821) (end 142.811179 126.299) (width 0.2) (layer "B.Cu") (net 4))
 (segment (start 138.25 105.25) (end 135.5 102.5) (width 0.2) (layer "B.Cu") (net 4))
 (segment (start 134.476 126.299) (end 128.015 132.76) (width 0.2) (layer "B.Cu") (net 4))
 (segment (start 149.985 132.76) (end 149.985 135.5) (width 0.2) (layer "B.Cu") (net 4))
 (segment (start 145.75 105.25) (end 138.25 105.25) (width 0.2) (layer "B.Cu") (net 4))
 (segment (start 145.75 105.25) (end 145.75 128.525) (width 0.2) (layer "B.Cu") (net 4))
 (segment (start 153.31 97.69) (end 145.75 105.25) (width 0.2) (layer "B.Cu") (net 4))
 (segment (start 145.225 81) (end 133 81) (width 0.2) (layer "B.Cu") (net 1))
 (segment (start 135.38876 108.301) (end 134.251 108.301) (width 0.2) (layer "B.Cu") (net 1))
 (segment (start 127.079 124.00876) (end 138.611 112.47676) (width 0.2) (layer "B.Cu") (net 1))
 (segment (start 138.611 112.47676) (end 138.611 111.52324) (width 0.2) (layer "B.Cu") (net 1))
 (segment (start 136.159 138.341) (end 127.079 138.341) (width 0.2) (layer "B.Cu") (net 1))
 (segment (start 133 81) (end 133 87.83) (width 0.2) (layer "B.Cu") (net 1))
 (segment (start 138.611 111.52324) (end 135.38876 108.301) (width 0.2) (layer "B.Cu") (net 1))
 (segment (start 139 135.5) (end 136.159 138.341) (width 0.2) (layer "B.Cu") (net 1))
 (segment (start 116.5 97.44) (end 123.39 97.44) (width 0.2) (layer "B.Cu") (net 1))
 (segment (start 127.079 138.341) (end 127.079 124.00876) (width 0.2) (layer "B.Cu") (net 1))
 (segment (start 123.39 97.44) (end 131.95 106) (width 0.2) (layer "B.Cu") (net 1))
 (segment (start 133 87.83) (end 123.39 97.44) (width 0.2) (layer "B.Cu") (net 1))
 (segment (start 134.251 108.301) (end 131.95 106) (width 0.2) (layer "B.Cu") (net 1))
 (segment (start 162.351 95.586) (end 147.765 81) (width 0.2) (layer "B.Cu") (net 2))
 (segment (start 162.351 98.14605) (end 162.351 95.586) (width 0.2) (layer "B.Cu") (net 2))
 (segment (start 155.24705 105.25) (end 162.351 98.14605) (width 0.2) (layer "B.Cu") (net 2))
 (segment (start 130.46 81) (end 131.661 79.799) (width 0.2) (layer "B.Cu") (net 2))
 (segment (start 131.661 79.799) (end 146.564 79.799) (width 0.2) (layer "B.Cu") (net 2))
 (segment (start 146.564 79.799) (end 147.765 81) (width 0.2) (layer "B.Cu") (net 2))
 (segment (start 148.29 105.25) (end 155.24705 105.25) (width 0.2) (layer "B.Cu") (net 2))
 (segment (start 137.46 112) (end 123.44 112) (width 0.2) (layer "B.Cu") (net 6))
 (segment (start 123.44 112) (end 116.5 105.06) (width 0.2) (layer "B.Cu") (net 6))
 (segment (start 140 112) (end 140 111.5) (width 0.2) (layer "B.Cu") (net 5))
 (segment (start 140 109) (end 142 107) (width 0.2) (layer "B.Cu") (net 5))
 (segment (start 140 112) (end 140 109) (width 0.2) (layer "B.Cu") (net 5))
 (segment (start 140 111.5) (end 135.5 107) (width 0.2) (layer "B.Cu") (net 5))
 (segment (start 115.399 94.362529) (end 115.399 97.89605) (width 0.2) (layer "B.Cu") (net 3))
 (segment (start 147.861471 79.398) (end 130.363529 79.398) (width 0.2) (layer "B.Cu") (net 3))
 (segment (start 162.752 98.31215) (end 162.752 94.288529) (width 0.2) (layer "B.Cu") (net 3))
 (segment (start 147.02 106.52) (end 154.54415 106.52) (width 0.2) (layer "B.Cu") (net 3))
 (segment (start 130.363529 79.398) (end 115.399 94.362529) (width 0.2) (layer "B.Cu") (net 3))
 (segment (start 115.399 97.89605) (end 123.50295 106) (width 0.2) (layer "B.Cu") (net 3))
 (segment (start 160.04 106.52) (end 147.02 106.52) (width 0.2) (layer "B.Cu") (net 3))
 (segment (start 154.54415 106.52) (end 162.752 98.31215) (width 0.2) (layer "B.Cu") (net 3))
 (segment (start 162.752 94.288529) (end 147.861471 79.398) (width 0.2) (layer "B.Cu") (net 3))
 (segment (start 123.50295 106) (end 128.55 106) (width 0.2) (layer "B.Cu") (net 3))
 (segment (start 161.25 105.31) (end 160.04 106.52) (width 0.2) (layer "B.Cu") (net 3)))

